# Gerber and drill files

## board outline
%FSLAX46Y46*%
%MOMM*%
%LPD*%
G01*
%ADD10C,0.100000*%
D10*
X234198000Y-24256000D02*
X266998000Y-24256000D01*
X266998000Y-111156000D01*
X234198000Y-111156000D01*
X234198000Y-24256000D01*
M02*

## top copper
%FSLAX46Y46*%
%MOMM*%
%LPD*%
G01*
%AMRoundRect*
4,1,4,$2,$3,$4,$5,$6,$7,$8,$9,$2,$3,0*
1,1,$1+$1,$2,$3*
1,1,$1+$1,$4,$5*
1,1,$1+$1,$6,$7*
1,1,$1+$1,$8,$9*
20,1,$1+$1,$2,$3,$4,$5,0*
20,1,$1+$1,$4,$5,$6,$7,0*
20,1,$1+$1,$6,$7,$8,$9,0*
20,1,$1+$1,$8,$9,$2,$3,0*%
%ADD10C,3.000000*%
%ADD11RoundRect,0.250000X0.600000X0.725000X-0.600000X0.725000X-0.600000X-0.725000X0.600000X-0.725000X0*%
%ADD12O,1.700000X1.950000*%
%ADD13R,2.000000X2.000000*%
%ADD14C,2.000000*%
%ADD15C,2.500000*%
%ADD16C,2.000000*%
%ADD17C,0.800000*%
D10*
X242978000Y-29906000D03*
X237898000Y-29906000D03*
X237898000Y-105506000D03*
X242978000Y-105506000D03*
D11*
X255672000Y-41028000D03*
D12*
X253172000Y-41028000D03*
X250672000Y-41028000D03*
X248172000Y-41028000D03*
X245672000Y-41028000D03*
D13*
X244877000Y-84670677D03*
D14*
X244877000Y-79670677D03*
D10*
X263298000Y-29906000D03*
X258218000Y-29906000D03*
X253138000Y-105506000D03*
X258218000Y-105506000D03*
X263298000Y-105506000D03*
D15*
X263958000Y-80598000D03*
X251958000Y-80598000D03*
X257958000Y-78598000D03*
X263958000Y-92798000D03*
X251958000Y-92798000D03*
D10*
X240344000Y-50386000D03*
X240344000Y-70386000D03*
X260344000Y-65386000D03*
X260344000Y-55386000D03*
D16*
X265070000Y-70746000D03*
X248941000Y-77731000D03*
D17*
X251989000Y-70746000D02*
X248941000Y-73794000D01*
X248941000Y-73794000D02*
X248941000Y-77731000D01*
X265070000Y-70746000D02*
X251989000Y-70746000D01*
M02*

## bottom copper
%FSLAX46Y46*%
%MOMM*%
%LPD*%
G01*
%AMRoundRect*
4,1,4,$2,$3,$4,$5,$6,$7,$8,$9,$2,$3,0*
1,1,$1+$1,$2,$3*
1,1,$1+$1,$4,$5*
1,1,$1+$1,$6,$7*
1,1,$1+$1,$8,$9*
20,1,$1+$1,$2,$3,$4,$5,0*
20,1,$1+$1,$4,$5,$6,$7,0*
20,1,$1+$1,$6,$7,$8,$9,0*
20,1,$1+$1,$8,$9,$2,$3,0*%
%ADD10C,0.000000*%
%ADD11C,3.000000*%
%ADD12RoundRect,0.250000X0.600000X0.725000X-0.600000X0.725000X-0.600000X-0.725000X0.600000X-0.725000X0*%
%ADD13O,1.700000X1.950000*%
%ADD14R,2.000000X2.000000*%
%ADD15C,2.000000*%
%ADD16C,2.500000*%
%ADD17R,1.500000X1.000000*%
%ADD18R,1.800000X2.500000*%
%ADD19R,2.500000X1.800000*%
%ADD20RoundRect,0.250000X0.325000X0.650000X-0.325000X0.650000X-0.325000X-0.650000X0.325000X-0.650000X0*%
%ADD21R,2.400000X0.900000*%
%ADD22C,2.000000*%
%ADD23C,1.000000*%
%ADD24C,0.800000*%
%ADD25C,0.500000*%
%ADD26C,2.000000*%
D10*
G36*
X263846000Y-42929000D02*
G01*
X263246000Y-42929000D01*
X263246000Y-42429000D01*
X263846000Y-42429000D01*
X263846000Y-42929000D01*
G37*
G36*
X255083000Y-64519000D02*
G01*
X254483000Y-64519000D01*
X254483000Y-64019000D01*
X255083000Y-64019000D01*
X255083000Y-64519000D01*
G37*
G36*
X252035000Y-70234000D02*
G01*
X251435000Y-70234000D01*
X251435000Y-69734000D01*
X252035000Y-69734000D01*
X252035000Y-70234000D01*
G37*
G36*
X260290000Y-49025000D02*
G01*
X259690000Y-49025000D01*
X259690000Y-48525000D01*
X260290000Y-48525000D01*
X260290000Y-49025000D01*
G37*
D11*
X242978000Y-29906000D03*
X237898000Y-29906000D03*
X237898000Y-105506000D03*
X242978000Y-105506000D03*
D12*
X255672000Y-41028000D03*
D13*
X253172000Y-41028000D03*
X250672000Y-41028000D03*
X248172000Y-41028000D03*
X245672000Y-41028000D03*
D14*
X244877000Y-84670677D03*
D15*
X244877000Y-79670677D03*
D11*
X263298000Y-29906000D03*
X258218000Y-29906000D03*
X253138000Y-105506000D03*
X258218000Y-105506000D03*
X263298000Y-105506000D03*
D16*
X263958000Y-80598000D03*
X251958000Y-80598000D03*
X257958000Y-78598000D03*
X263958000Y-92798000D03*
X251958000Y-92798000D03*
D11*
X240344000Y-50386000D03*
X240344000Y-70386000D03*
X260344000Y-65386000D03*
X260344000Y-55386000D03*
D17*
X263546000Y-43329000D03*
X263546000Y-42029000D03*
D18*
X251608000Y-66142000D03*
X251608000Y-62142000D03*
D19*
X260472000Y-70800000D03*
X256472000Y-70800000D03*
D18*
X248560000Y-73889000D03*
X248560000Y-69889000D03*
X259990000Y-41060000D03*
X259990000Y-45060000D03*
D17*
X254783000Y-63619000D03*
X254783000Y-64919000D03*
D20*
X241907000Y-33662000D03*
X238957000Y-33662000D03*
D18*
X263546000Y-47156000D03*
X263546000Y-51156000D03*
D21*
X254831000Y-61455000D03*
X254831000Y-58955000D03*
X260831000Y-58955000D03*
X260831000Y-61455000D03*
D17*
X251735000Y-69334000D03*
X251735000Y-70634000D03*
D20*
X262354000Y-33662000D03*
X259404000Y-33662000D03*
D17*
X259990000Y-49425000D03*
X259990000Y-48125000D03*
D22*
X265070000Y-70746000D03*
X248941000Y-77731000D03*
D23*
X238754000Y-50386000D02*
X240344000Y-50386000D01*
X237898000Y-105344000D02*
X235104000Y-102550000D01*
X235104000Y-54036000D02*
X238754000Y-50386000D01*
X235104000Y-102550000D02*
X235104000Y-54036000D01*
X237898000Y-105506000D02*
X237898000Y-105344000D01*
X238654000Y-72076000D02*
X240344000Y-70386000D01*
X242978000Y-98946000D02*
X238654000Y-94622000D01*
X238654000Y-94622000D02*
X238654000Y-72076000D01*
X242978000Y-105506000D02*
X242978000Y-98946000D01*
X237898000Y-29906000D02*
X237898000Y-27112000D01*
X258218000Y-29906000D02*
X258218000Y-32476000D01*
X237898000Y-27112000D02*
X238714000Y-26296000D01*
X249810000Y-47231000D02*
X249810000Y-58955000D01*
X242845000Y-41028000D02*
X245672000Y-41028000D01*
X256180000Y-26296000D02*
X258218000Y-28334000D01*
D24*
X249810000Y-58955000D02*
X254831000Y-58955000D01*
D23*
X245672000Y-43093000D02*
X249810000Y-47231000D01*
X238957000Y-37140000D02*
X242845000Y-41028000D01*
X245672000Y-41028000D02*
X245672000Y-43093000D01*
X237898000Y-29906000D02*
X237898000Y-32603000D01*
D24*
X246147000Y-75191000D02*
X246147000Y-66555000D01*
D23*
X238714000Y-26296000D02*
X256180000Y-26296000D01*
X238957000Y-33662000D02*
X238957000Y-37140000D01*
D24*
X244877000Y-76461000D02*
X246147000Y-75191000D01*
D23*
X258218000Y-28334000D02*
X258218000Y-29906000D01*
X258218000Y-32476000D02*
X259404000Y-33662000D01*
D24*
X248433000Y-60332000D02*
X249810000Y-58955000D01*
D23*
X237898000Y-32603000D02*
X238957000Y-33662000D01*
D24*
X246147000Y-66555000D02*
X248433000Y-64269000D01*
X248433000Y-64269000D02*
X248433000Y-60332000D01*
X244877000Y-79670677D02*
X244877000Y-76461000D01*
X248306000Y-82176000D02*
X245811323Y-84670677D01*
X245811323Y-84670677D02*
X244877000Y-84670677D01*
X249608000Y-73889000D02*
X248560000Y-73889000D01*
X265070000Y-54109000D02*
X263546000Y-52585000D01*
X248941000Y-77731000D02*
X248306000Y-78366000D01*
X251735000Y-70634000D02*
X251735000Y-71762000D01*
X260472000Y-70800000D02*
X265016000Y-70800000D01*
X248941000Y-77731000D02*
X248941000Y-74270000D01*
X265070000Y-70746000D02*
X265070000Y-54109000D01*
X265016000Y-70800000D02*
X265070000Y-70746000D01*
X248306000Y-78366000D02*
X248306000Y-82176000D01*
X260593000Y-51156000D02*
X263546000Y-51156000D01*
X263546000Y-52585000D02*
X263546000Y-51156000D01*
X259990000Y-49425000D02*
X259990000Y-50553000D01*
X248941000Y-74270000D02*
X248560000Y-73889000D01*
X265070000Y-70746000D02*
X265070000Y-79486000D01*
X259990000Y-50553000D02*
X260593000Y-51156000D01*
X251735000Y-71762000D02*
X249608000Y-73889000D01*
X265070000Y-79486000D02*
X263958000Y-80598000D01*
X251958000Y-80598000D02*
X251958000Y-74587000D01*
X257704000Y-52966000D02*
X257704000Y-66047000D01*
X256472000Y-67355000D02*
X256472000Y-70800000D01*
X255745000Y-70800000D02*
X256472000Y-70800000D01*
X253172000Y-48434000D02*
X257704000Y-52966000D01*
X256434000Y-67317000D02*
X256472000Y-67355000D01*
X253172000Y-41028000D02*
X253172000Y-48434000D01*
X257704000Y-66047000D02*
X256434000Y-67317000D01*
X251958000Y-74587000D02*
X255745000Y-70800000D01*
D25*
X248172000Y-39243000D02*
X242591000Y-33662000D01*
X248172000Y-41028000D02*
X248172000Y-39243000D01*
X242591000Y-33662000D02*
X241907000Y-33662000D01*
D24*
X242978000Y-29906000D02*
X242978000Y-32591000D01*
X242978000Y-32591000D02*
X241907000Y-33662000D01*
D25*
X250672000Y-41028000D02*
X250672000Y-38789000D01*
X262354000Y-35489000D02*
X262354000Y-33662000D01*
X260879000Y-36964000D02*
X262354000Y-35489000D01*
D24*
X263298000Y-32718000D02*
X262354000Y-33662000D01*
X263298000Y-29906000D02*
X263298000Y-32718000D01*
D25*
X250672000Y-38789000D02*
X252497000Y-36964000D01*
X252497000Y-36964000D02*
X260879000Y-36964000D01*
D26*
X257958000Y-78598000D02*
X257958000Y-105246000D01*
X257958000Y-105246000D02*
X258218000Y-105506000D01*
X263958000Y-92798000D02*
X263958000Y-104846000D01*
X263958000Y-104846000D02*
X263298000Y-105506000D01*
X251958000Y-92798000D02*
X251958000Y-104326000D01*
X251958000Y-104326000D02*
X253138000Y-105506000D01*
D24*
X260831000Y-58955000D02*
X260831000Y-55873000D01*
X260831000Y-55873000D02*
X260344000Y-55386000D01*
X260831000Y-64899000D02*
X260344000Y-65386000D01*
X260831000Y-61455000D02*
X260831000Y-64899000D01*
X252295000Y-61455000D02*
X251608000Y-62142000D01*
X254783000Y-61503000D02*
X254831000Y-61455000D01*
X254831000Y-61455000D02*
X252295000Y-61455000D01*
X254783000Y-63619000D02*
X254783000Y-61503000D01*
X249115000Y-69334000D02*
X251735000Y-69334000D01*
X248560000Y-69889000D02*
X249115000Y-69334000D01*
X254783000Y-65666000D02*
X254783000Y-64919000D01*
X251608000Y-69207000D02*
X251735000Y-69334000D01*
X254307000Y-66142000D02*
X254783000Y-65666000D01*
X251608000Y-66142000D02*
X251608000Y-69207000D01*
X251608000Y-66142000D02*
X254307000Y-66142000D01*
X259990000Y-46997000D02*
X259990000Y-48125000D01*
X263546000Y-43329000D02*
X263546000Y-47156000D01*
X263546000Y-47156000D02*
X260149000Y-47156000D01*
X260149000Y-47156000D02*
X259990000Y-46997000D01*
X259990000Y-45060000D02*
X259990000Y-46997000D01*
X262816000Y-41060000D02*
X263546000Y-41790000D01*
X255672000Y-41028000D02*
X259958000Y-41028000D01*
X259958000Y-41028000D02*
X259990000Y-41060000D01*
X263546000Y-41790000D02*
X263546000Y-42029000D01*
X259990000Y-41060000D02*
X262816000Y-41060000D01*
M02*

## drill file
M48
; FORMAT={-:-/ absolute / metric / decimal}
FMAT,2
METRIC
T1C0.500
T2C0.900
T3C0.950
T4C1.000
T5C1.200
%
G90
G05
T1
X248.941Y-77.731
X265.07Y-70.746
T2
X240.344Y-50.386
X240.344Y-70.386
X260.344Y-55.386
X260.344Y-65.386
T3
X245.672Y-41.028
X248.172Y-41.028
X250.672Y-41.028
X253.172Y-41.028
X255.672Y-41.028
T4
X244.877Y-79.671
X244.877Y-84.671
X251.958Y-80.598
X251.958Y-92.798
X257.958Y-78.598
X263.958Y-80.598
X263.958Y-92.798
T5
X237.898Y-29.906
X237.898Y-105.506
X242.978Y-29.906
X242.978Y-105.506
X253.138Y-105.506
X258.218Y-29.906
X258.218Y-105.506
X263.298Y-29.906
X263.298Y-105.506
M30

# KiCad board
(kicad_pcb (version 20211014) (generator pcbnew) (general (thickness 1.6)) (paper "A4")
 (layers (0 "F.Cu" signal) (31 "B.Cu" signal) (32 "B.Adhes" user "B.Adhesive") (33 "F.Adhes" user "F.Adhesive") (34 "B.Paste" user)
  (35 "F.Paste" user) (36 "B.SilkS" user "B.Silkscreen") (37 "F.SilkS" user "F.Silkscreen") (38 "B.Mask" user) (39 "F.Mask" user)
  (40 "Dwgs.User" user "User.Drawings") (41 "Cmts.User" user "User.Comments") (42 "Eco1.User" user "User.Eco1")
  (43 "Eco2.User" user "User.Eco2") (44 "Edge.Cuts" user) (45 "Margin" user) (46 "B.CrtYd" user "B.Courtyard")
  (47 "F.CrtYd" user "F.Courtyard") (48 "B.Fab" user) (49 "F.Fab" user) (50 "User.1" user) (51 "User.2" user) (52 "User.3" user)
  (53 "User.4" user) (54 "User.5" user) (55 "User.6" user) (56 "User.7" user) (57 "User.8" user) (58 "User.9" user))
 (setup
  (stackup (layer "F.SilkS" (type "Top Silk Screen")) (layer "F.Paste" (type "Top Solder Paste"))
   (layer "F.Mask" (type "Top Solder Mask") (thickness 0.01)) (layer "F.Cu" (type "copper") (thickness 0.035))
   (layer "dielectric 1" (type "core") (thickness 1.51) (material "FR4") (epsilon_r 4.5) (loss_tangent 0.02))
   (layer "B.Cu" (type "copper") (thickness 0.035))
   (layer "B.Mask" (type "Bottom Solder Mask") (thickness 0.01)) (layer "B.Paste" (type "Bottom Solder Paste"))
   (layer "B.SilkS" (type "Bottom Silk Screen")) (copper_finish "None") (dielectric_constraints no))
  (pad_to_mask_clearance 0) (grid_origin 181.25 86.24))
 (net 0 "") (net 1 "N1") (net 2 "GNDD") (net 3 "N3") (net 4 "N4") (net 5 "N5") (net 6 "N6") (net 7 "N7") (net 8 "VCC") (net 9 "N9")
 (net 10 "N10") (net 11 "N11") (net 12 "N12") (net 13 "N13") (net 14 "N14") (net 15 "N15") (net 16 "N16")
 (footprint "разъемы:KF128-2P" (layer "F.Cu") (at 240.438 29.906 180)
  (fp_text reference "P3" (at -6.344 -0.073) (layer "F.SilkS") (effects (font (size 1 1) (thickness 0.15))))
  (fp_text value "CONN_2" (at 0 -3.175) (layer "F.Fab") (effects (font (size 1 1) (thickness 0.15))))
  (pad "1" thru_hole circle locked (at -2.54 0 180) (size 3 3) (drill 1.2) (layers *.Cu *.Mask "F.SilkS") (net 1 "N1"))
  (pad "2" thru_hole circle locked (at 2.54 0 180) (size 3 3) (drill 1.2) (layers *.Cu *.Mask "F.SilkS") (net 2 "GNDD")))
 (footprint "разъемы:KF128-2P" (layer "F.Cu") (at 240.438 105.506)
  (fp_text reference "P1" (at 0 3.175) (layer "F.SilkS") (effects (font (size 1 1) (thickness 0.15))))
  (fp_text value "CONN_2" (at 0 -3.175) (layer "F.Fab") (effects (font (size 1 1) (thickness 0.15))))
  (pad "1" thru_hole circle locked (at -2.54 0) (size 3 3) (drill 1.2) (layers *.Cu *.Mask "F.SilkS") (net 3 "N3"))
  (pad "2" thru_hole circle locked (at 2.54 0) (size 3 3) (drill 1.2) (layers *.Cu *.Mask "F.SilkS") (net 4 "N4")))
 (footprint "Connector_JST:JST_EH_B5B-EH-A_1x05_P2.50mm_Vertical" (layer "F.Cu") (at 255.672 41.028 180)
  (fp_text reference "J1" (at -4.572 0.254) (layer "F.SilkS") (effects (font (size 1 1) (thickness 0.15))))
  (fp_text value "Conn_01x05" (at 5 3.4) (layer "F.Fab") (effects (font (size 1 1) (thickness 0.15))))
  (pad "1" thru_hole roundrect (at 0 0 180) (size 1.7 1.95) (drill 0.95) (layers *.Cu *.Mask) (roundrect_rratio 0.1470588235) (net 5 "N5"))
  (pad "2" thru_hole oval (at 2.5 0 180) (size 1.7 1.95) (drill 0.95) (layers *.Cu *.Mask) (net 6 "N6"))
  (pad "3" thru_hole oval (at 5 0 180) (size 1.7 1.95) (drill 0.95) (layers *.Cu *.Mask) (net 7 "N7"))
  (pad "4" thru_hole oval (at 7.5 0 180) (size 1.7 1.95) (drill 0.95) (layers *.Cu *.Mask) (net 1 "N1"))
  (pad "5" thru_hole oval (at 10 0 180) (size 1.7 1.95) (drill 0.95) (layers *.Cu *.Mask) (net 2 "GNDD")))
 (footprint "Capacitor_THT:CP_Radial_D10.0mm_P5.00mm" (layer "F.Cu") (at 244.877 84.670677 90)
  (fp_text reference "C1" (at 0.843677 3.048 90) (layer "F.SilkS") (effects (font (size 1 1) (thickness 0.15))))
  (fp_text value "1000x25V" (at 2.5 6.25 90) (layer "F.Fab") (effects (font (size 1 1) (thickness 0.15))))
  (pad "1" thru_hole rect (at 0 0 90) (size 2 2) (drill 1) (layers *.Cu *.Mask) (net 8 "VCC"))
  (pad "2" thru_hole circle (at 5 0 90) (size 2 2) (drill 1) (layers *.Cu *.Mask) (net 2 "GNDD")))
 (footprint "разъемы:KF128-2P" (layer "F.Cu") (at 260.758 29.906 180)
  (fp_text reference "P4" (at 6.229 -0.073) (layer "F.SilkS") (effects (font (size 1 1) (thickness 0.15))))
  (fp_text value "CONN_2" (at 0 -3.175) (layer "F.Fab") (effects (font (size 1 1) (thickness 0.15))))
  (pad "1" thru_hole circle locked (at -2.54 0 180) (size 3 3) (drill 1.2) (layers *.Cu *.Mask "F.SilkS") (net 7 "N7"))
  (pad "2" thru_hole circle locked (at 2.54 0 180) (size 3 3) (drill 1.2) (layers *.Cu *.Mask "F.SilkS") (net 2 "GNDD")))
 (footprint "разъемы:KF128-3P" (layer "F.Cu") (at 258.218 105.506)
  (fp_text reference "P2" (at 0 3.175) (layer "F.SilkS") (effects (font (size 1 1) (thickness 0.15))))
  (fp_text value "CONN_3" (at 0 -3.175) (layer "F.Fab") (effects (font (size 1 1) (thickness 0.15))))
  (pad "1" thru_hole circle locked (at -5.08 0) (size 3 3) (drill 1.2) (layers *.Cu *.Mask "F.SilkS") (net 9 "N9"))
  (pad "2" thru_hole circle locked (at 0 0) (size 3 3) (drill 1.2) (layers *.Cu *.Mask "F.SilkS") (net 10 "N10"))
  (pad "3" thru_hole circle locked (at 5.08 0) (size 3 3) (drill 1.2) (layers *.Cu *.Mask "F.SilkS") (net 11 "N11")))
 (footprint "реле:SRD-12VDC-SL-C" (layer "F.Cu") (at 257.958 86.748 -90)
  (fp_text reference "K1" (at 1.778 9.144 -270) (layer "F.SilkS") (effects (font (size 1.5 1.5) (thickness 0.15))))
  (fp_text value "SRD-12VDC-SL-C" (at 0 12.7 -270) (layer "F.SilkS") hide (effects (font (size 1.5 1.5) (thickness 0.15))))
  (pad "1" thru_hole circle locked (at -6.15 -6) (size 2.5 2.5) (drill 1) (layers *.Cu *.Mask "F.SilkS") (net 8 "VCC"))
  (pad "2" thru_hole circle locked (at -6.15 6) (size 2.5 2.5) (drill 1) (layers *.Cu *.Mask "F.SilkS") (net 6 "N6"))
  (pad "3" thru_hole circle locked (at -8.15 0) (size 2.5 2.5) (drill 1) (layers *.Cu *.Mask "F.SilkS") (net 10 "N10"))
  (pad "4" thru_hole circle locked (at 6.05 -6) (size 2.5 2.5) (drill 1) (layers *.Cu *.Mask "F.SilkS") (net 11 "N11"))
  (pad "5" thru_hole circle locked (at 6.05 6) (size 2.5 2.5) (drill 1) (layers *.Cu *.Mask "F.SilkS") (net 9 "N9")))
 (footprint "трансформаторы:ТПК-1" (layer "F.Cu") (at 250.344 60.386 -90)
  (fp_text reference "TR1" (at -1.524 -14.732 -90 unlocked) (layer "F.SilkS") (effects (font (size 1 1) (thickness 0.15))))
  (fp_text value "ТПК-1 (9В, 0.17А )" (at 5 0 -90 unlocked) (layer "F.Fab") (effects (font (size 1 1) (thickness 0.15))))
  (pad "1" thru_hole circle (at -10 10 270) (size 3 3) (drill 0.9) (layers *.Cu *.Mask) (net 3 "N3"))
  (pad "5" thru_hole circle (at 10 10 270) (size 3 3) (drill 0.9) (layers *.Cu *.Mask) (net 4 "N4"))
  (pad "7" thru_hole circle (at 5 -10 270) (size 3 3) (drill 0.9) (layers *.Cu *.Mask) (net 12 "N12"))
  (pad "9" thru_hole circle (at -5 -10 270) (size 3 3) (drill 0.9) (layers *.Cu *.Mask) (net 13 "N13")))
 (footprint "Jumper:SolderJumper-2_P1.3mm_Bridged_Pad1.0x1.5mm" (layer "B.Cu") (at 263.546 42.679 90)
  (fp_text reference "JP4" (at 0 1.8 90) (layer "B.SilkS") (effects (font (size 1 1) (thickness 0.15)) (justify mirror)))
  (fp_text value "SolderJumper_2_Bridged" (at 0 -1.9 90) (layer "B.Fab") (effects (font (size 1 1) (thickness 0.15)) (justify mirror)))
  (fp_poly (pts (xy -0.25 0.3) (xy 0.25 0.3) (xy 0.25 -0.3) (xy -0.25 -0.3)) (layer "B.Cu") (width 0) (fill solid))
  (pad "1" smd rect (at -0.65 0 90) (size 1 1.5) (layers "B.Cu" "B.Mask") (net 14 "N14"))
  (pad "2" smd rect (at 0.65 0 90) (size 1 1.5) (layers "B.Cu" "B.Mask") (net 5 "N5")))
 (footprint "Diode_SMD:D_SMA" (layer "B.Cu") (at 251.608 64.142 90)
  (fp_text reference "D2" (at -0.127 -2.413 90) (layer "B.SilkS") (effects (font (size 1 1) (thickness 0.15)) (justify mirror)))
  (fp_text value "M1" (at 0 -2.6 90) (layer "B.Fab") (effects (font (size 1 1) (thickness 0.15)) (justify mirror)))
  (pad "1" smd rect (at -2 0 90) (size 2.5 1.8) (layers "B.Cu" "B.Paste" "B.Mask") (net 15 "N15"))
  (pad "2" smd rect (at 2 0 90) (size 2.5 1.8) (layers "B.Cu" "B.Paste" "B.Mask") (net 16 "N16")))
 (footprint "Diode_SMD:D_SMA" (layer "B.Cu") (at 258.472 70.8 180)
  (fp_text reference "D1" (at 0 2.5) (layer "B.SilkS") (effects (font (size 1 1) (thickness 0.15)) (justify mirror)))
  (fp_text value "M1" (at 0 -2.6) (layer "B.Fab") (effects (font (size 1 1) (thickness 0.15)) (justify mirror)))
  (pad "1" smd rect (at -2 0 180) (size 2.5 1.8) (layers "B.Cu" "B.Paste" "B.Mask") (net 8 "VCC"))
  (pad "2" smd rect (at 2 0 180) (size 2.5 1.8) (layers "B.Cu" "B.Paste" "B.Mask") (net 6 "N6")))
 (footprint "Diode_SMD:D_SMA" (layer "B.Cu") (at 248.56 71.889 90)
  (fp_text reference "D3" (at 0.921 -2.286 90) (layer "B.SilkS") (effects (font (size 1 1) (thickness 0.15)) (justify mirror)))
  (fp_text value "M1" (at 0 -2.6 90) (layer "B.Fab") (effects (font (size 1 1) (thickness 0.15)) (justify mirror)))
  (pad "1" smd rect (at -2 0 90) (size 2.5 1.8) (layers "B.Cu" "B.Paste" "B.Mask") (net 8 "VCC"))
  (pad "2" smd rect (at 2 0 90) (size 2.5 1.8) (layers "B.Cu" "B.Paste" "B.Mask") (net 15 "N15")))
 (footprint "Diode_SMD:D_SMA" (layer "B.Cu") (at 259.99 43.06 -90)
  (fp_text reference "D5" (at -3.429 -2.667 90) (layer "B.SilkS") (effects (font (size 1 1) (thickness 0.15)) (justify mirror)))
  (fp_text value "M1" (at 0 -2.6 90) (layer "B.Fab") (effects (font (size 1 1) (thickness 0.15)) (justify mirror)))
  (pad "1" smd rect (at -2 0 270) (size 2.5 1.8) (layers "B.Cu" "B.Paste" "B.Mask") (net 5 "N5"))
  (pad "2" smd rect (at 2 0 270) (size 2.5 1.8) (layers "B.Cu" "B.Paste" "B.Mask") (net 14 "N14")))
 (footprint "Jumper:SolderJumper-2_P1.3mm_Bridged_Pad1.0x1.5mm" (layer "B.Cu") (at 254.783 64.269 -90)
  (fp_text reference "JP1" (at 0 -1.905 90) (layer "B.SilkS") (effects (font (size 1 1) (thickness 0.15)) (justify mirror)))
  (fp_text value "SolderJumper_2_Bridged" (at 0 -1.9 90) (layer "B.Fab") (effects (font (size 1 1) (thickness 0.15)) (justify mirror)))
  (fp_poly (pts (xy -0.25 0.3) (xy 0.25 0.3) (xy 0.25 -0.3) (xy -0.25 -0.3)) (layer "B.Cu") (width 0) (fill solid))
  (pad "1" smd rect (at -0.65 0 270) (size 1 1.5) (layers "B.Cu" "B.Mask") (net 16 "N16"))
  (pad "2" smd rect (at 0.65 0 270) (size 1 1.5) (layers "B.Cu" "B.Mask") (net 15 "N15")))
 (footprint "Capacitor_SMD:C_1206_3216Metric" (layer "B.Cu") (at 240.432 33.662 180)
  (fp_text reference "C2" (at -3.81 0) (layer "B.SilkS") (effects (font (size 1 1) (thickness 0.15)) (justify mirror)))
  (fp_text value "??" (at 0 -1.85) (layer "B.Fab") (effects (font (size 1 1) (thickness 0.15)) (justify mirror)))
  (pad "1" smd roundrect (at -1.475 0 180) (size 1.15 1.8) (layers "B.Cu" "B.Paste" "B.Mask") (roundrect_rratio 0.2173913043) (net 1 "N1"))
  (pad "2" smd roundrect (at 1.475 0 180) (size 1.15 1.8) (layers "B.Cu" "B.Paste" "B.Mask") (roundrect_rratio 0.2173913043) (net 2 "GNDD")))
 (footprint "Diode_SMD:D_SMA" (layer "B.Cu") (at 263.546 49.156 -90)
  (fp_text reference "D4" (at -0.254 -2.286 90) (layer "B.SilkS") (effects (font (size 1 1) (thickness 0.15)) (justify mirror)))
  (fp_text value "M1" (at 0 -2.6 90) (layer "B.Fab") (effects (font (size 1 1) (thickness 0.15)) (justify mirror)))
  (pad "1" smd rect (at -2 0 270) (size 2.5 1.8) (layers "B.Cu" "B.Paste" "B.Mask") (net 14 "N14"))
  (pad "2" smd rect (at 2 0 270) (size 2.5 1.8) (layers "B.Cu" "B.Paste" "B.Mask") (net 8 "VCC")))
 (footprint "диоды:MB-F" (layer "B.Cu") (at 257.831 60.205)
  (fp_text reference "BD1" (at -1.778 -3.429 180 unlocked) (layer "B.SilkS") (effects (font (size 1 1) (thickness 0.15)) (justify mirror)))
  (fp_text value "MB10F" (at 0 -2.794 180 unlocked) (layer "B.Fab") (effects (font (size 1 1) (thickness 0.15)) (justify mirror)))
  (pad "1" smd rect (at -3 1.25) (size 2.4 0.9) (layers "B.Cu" "B.Paste" "B.Mask") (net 16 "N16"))
  (pad "2" smd rect (at -3 -1.25) (size 2.4 0.9) (layers "B.Cu" "B.Paste" "B.Mask") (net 2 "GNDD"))
  (pad "3" smd rect (at 3 -1.25) (size 2.4 0.9) (layers "B.Cu" "B.Paste" "B.Mask") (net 13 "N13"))
  (pad "4" smd rect (at 3 1.25) (size 2.4 0.9) (layers "B.Cu" "B.Paste" "B.Mask") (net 12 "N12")))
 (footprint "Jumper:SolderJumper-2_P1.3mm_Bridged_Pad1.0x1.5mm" (layer "B.Cu") (at 251.735 69.984 -90)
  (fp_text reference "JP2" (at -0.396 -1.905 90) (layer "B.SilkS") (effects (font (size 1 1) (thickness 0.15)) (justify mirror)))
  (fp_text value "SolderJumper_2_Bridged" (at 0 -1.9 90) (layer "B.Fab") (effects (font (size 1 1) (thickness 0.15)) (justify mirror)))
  (fp_poly (pts (xy -0.25 0.3) (xy 0.25 0.3) (xy 0.25 -0.3) (xy -0.25 -0.3)) (layer "B.Cu") (width 0) (fill solid))
  (pad "1" smd rect (at -0.65 0 270) (size 1 1.5) (layers "B.Cu" "B.Mask") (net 15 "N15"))
  (pad "2" smd rect (at 0.65 0 270) (size 1 1.5) (layers "B.Cu" "B.Mask") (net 8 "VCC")))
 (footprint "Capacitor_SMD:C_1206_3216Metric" (layer "B.Cu") (at 260.879 33.662 180)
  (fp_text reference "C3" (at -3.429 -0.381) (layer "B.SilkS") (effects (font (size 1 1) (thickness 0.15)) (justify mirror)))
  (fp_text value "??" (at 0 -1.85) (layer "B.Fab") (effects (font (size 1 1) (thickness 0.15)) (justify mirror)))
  (pad "1" smd roundrect (at -1.475 0 180) (size 1.15 1.8) (layers "B.Cu" "B.Paste" "B.Mask") (roundrect_rratio 0.2173913043) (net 7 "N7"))
  (pad "2" smd roundrect (at 1.475 0 180) (size 1.15 1.8) (layers "B.Cu" "B.Paste" "B.Mask") (roundrect_rratio 0.2173913043) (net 2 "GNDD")))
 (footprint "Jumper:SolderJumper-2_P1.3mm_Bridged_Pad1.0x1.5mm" (layer "B.Cu") (at 259.99 48.775 90)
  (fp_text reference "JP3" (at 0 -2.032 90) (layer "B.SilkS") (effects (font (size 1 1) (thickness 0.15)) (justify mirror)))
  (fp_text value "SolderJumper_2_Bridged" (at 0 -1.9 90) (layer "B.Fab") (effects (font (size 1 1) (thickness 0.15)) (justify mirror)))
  (fp_poly (pts (xy -0.25 0.3) (xy 0.25 0.3) (xy 0.25 -0.3) (xy -0.25 -0.3)) (layer "B.Cu") (width 0) (fill solid))
  (pad "1" smd rect (at -0.65 0 90) (size 1 1.5) (layers "B.Cu" "B.Mask") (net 8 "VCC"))
  (pad "2" smd rect (at 0.65 0 90) (size 1 1.5) (layers "B.Cu" "B.Mask") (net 14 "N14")))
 (gr_rect (start 234.198 111.156) (end 266.998 24.256) (layer "Edge.Cuts") (width 0.1) (fill none))
 (segment (start 238.754 50.386) (end 240.344 50.386) (width 1) (layer "B.Cu") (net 3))
 (segment (start 237.898 105.344) (end 235.104 102.55) (width 1) (layer "B.Cu") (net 3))
 (segment (start 235.104 54.036) (end 238.754 50.386) (width 1) (layer "B.Cu") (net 3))
 (segment (start 235.104 102.55) (end 235.104 54.036) (width 1) (layer "B.Cu") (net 3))
 (segment (start 237.898 105.506) (end 237.898 105.344) (width 1) (layer "B.Cu") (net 3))
 (segment (start 238.654 72.076) (end 240.344 70.386) (width 1) (layer "B.Cu") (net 4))
 (segment (start 242.978 98.946) (end 238.654 94.622) (width 1) (layer "B.Cu") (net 4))
 (segment (start 238.654 94.622) (end 238.654 72.076) (width 1) (layer "B.Cu") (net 4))
 (segment (start 242.978 105.506) (end 242.978 98.946) (width 1) (layer "B.Cu") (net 4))
 (segment (start 237.898 29.906) (end 237.898 27.112) (width 1) (layer "B.Cu") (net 2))
 (segment (start 258.218 29.906) (end 258.218 32.476) (width 1) (layer "B.Cu") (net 2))
 (segment (start 237.898 27.112) (end 238.714 26.296) (width 1) (layer "B.Cu") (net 2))
 (segment (start 249.81 47.231) (end 249.81 58.955) (width 1) (layer "B.Cu") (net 2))
 (segment (start 242.845 41.028) (end 245.672 41.028) (width 1) (layer "B.Cu") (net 2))
 (segment (start 256.18 26.296) (end 258.218 28.334) (width 1) (layer "B.Cu") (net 2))
 (segment (start 249.81 58.955) (end 254.831 58.955) (width 0.8) (layer "B.Cu") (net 2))
 (segment (start 245.672 43.093) (end 249.81 47.231) (width 1) (layer "B.Cu") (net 2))
 (segment (start 238.957 37.14) (end 242.845 41.028) (width 1) (layer "B.Cu") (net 2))
 (segment (start 245.672 41.028) (end 245.672 43.093) (width 1) (layer "B.Cu") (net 2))
 (segment (start 237.898 29.906) (end 237.898 32.603) (width 1) (layer "B.Cu") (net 2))
 (segment (start 246.147 75.191) (end 246.147 66.555) (width 0.8) (layer "B.Cu") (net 2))
 (segment (start 238.714 26.296) (end 256.18 26.296) (width 1) (layer "B.Cu") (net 2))
 (segment (start 238.957 33.662) (end 238.957 37.14) (width 1) (layer "B.Cu") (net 2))
 (segment (start 244.877 76.461) (end 246.147 75.191) (width 0.8) (layer "B.Cu") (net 2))
 (segment (start 258.218 28.334) (end 258.218 29.906) (width 1) (layer "B.Cu") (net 2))
 (segment (start 258.218 32.476) (end 259.404 33.662) (width 1) (layer "B.Cu") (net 2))
 (segment (start 248.433 60.332) (end 249.81 58.955) (width 0.8) (layer "B.Cu") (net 2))
 (segment (start 237.898 32.603) (end 238.957 33.662) (width 1) (layer "B.Cu") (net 2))
 (segment (start 246.147 66.555) (end 248.433 64.269) (width 0.8) (layer "B.Cu") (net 2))
 (segment (start 248.433 64.269) (end 248.433 60.332) (width 0.8) (layer "B.Cu") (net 2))
 (segment (start 244.877 79.670677) (end 244.877 76.461) (width 0.8) (layer "B.Cu") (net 2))
 (segment (start 251.989 70.746) (end 248.941 73.794) (width 0.8) (layer "F.Cu") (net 8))
 (segment (start 248.941 73.794) (end 248.941 77.731) (width 0.8) (layer "F.Cu") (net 8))
 (segment (start 265.07 70.746) (end 251.989 70.746) (width 0.8) (layer "F.Cu") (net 8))
 (via (at 265.07 70.746) (size 2) (drill 0.5) (layers "F.Cu" "B.Cu") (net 8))
 (via (at 248.941 77.731) (size 2) (drill 0.5) (layers "F.Cu" "B.Cu") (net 8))
 (segment (start 248.306 82.176) (end 245.811323 84.670677) (width 0.8) (layer "B.Cu") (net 8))
 (segment (start 245.811323 84.670677) (end 244.877 84.670677) (width 0.8) (layer "B.Cu") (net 8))
 (segment (start 249.608 73.889) (end 248.56 73.889) (width 0.8) (layer "B.Cu") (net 8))
 (segment (start 265.07 54.109) (end 263.546 52.585) (width 0.8) (layer "B.Cu") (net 8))
 (segment (start 248.941 77.731) (end 248.306 78.366) (width 0.8) (layer "B.Cu") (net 8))
 (segment (start 251.735 70.634) (end 251.735 71.762) (width 0.8) (layer "B.Cu") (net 8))
 (segment (start 260.472 70.8) (end 265.016 70.8) (width 0.8) (layer "B.Cu") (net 8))
 (segment (start 248.941 77.731) (end 248.941 74.27) (width 0.8) (layer "B.Cu") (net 8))
 (segment (start 265.07 70.746) (end 265.07 54.109) (width 0.8) (layer "B.Cu") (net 8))
 (segment (start 265.016 70.8) (end 265.07 70.746) (width 0.8) (layer "B.Cu") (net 8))
 (segment (start 248.306 78.366) (end 248.306 82.176) (width 0.8) (layer "B.Cu") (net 8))
 (segment (start 260.593 51.156) (end 263.546 51.156) (width 0.8) (layer "B.Cu") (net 8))
 (segment (start 263.546 52.585) (end 263.546 51.156) (width 0.8) (layer "B.Cu") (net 8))
 (segment (start 259.99 49.425) (end 259.99 50.553) (width 0.8) (layer "B.Cu") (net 8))
 (segment (start 248.941 74.27) (end 248.56 73.889) (width 0.8) (layer "B.Cu") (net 8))
 (segment (start 265.07 70.746) (end 265.07 79.486) (width 0.8) (layer "B.Cu") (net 8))
 (segment (start 259.99 50.553) (end 260.593 51.156) (width 0.8) (layer "B.Cu") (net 8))
 (segment (start 251.735 71.762) (end 249.608 73.889) (width 0.8) (layer "B.Cu") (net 8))
 (segment (start 265.07 79.486) (end 263.958 80.598) (width 0.8) (layer "B.Cu") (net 8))
 (segment (start 251.958 80.598) (end 251.958 74.587) (width 0.8) (layer "B.Cu") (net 6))
 (segment (start 257.704 52.966) (end 257.704 66.047) (width 0.8) (layer "B.Cu") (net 6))
 (segment (start 256.472 67.355) (end 256.472 70.8) (width 0.8) (layer "B.Cu") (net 6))
 (segment (start 255.745 70.8) (end 256.472 70.8) (width 0.8) (layer "B.Cu") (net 6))
 (segment (start 253.172 48.434) (end 257.704 52.966) (width 0.8) (layer "B.Cu") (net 6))
 (segment (start 256.434 67.317) (end 256.472 67.355) (width 0.8) (layer "B.Cu") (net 6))
 (segment (start 253.172 41.028) (end 253.172 48.434) (width 0.8) (layer "B.Cu") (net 6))
 (segment (start 257.704 66.047) (end 256.434 67.317) (width 0.8) (layer "B.Cu") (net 6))
 (segment (start 251.958 74.587) (end 255.745 70.8) (width 0.8) (layer "B.Cu") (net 6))
 (segment (start 248.172 39.243) (end 242.591 33.662) (width 0.5) (layer "B.Cu") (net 1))
 (segment (start 248.172 41.028) (end 248.172 39.243) (width 0.5) (layer "B.Cu") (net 1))
 (segment (start 242.591 33.662) (end 241.907 33.662) (width 0.5) (layer "B.Cu") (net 1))
 (segment (start 242.978 29.906) (end 242.978 32.591) (width 0.8) (layer "B.Cu") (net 1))
 (segment (start 242.978 32.591) (end 241.907 33.662) (width 0.8) (layer "B.Cu") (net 1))
 (segment (start 250.672 41.028) (end 250.672 38.789) (width 0.5) (layer "B.Cu") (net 7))
 (segment (start 262.354 35.489) (end 262.354 33.662) (width 0.5) (layer "B.Cu") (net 7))
 (segment (start 260.879 36.964) (end 262.354 35.489) (width 0.5) (layer "B.Cu") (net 7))
 (segment (start 263.298 32.718) (end 262.354 33.662) (width 0.8) (layer "B.Cu") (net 7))
 (segment (start 263.298 29.906) (end 263.298 32.718) (width 0.8) (layer "B.Cu") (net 7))
 (segment (start 250.672 38.789) (end 252.497 36.964) (width 0.5) (layer "B.Cu") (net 7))
 (segment (start 252.497 36.964) (end 260.879 36.964) (width 0.5) (layer "B.Cu") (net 7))
 (segment (start 257.958 78.598) (end 257.958 105.246) (width 2) (layer "B.Cu") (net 10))
 (segment (start 257.958 105.246) (end 258.218 105.506) (width 2) (layer "B.Cu") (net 10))
 (segment (start 263.958 92.798) (end 263.958 104.846) (width 2) (layer "B.Cu") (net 11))
 (segment (start 263.958 104.846) (end 263.298 105.506) (width 2) (layer "B.Cu") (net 11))
 (segment (start 251.958 92.798) (end 251.958 104.326) (width 2) (layer "B.Cu") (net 9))
 (segment (start 251.958 104.326) (end 253.138 105.506) (width 2) (layer "B.Cu") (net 9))
 (segment (start 260.831 58.955) (end 260.831 55.873) (width 0.8) (layer "B.Cu") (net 13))
 (segment (start 260.831 55.873) (end 260.344 55.386) (width 0.8) (layer "B.Cu") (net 13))
 (segment (start 260.831 64.899) (end 260.344 65.386) (width 0.8) (layer "B.Cu") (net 12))
 (segment (start 260.831 61.455) (end 260.831 64.899) (width 0.8) (layer "B.Cu") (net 12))
 (segment (start 252.295 61.455) (end 251.608 62.142) (width 0.8) (layer "B.Cu") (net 16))
 (segment (start 254.783 61.503) (end 254.831 61.455) (width 0.8) (layer "B.Cu") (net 16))
 (segment (start 254.831 61.455) (end 252.295 61.455) (width 0.8) (layer "B.Cu") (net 16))
 (segment (start 254.783 63.619) (end 254.783 61.503) (width 0.8) (layer "B.Cu") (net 16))
 (segment (start 249.115 69.334) (end 251.735 69.334) (width 0.8) (layer "B.Cu") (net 15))
 (segment (start 248.56 69.889) (end 249.115 69.334) (width 0.8) (layer "B.Cu") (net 15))
 (segment (start 254.783 65.666) (end 254.783 64.919) (width 0.8) (layer "B.Cu") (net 15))
 (segment (start 251.608 69.207) (end 251.735 69.334) (width 0.8) (layer "B.Cu") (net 15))
 (segment (start 254.307 66.142) (end 254.783 65.666) (width 0.8) (layer "B.Cu") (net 15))
 (segment (start 251.608 66.142) (end 251.608 69.207) (width 0.8) (layer "B.Cu") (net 15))
 (segment (start 251.608 66.142) (end 254.307 66.142) (width 0.8) (layer "B.Cu") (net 15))
 (segment (start 259.99 46.997) (end 259.99 48.125) (width 0.8) (layer "B.Cu") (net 14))
 (segment (start 263.546 43.329) (end 263.546 47.156) (width 0.8) (layer "B.Cu") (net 14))
 (segment (start 263.546 47.156) (end 260.149 47.156) (width 0.8) (layer "B.Cu") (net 14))
 (segment (start 260.149 47.156) (end 259.99 46.997) (width 0.8) (layer "B.Cu") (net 14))
 (segment (start 259.99 45.06) (end 259.99 46.997) (width 0.8) (layer "B.Cu") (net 14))
 (segment (start 262.816 41.06) (end 263.546 41.79) (width 0.8) (layer "B.Cu") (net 5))
 (segment (start 255.672 41.028) (end 259.958 41.028) (width 0.8) (layer "B.Cu") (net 5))
 (segment (start 259.958 41.028) (end 259.99 41.06) (width 0.8) (layer "B.Cu") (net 5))
 (segment (start 263.546 41.79) (end 263.546 42.029) (width 0.8) (layer "B.Cu") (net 5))
 (segment (start 259.99 41.06) (end 262.816 41.06) (width 0.8) (layer "B.Cu") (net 5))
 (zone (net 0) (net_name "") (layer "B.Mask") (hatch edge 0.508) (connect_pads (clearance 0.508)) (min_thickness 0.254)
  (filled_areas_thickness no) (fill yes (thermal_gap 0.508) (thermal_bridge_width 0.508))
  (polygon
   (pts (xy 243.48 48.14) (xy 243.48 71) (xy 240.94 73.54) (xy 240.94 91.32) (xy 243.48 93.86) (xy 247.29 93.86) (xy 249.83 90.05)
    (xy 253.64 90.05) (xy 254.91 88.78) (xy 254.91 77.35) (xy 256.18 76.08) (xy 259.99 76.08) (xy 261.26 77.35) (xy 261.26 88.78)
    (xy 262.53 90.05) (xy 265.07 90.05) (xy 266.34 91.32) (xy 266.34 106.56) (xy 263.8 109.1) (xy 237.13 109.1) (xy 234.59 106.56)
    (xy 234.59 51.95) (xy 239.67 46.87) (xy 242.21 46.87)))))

